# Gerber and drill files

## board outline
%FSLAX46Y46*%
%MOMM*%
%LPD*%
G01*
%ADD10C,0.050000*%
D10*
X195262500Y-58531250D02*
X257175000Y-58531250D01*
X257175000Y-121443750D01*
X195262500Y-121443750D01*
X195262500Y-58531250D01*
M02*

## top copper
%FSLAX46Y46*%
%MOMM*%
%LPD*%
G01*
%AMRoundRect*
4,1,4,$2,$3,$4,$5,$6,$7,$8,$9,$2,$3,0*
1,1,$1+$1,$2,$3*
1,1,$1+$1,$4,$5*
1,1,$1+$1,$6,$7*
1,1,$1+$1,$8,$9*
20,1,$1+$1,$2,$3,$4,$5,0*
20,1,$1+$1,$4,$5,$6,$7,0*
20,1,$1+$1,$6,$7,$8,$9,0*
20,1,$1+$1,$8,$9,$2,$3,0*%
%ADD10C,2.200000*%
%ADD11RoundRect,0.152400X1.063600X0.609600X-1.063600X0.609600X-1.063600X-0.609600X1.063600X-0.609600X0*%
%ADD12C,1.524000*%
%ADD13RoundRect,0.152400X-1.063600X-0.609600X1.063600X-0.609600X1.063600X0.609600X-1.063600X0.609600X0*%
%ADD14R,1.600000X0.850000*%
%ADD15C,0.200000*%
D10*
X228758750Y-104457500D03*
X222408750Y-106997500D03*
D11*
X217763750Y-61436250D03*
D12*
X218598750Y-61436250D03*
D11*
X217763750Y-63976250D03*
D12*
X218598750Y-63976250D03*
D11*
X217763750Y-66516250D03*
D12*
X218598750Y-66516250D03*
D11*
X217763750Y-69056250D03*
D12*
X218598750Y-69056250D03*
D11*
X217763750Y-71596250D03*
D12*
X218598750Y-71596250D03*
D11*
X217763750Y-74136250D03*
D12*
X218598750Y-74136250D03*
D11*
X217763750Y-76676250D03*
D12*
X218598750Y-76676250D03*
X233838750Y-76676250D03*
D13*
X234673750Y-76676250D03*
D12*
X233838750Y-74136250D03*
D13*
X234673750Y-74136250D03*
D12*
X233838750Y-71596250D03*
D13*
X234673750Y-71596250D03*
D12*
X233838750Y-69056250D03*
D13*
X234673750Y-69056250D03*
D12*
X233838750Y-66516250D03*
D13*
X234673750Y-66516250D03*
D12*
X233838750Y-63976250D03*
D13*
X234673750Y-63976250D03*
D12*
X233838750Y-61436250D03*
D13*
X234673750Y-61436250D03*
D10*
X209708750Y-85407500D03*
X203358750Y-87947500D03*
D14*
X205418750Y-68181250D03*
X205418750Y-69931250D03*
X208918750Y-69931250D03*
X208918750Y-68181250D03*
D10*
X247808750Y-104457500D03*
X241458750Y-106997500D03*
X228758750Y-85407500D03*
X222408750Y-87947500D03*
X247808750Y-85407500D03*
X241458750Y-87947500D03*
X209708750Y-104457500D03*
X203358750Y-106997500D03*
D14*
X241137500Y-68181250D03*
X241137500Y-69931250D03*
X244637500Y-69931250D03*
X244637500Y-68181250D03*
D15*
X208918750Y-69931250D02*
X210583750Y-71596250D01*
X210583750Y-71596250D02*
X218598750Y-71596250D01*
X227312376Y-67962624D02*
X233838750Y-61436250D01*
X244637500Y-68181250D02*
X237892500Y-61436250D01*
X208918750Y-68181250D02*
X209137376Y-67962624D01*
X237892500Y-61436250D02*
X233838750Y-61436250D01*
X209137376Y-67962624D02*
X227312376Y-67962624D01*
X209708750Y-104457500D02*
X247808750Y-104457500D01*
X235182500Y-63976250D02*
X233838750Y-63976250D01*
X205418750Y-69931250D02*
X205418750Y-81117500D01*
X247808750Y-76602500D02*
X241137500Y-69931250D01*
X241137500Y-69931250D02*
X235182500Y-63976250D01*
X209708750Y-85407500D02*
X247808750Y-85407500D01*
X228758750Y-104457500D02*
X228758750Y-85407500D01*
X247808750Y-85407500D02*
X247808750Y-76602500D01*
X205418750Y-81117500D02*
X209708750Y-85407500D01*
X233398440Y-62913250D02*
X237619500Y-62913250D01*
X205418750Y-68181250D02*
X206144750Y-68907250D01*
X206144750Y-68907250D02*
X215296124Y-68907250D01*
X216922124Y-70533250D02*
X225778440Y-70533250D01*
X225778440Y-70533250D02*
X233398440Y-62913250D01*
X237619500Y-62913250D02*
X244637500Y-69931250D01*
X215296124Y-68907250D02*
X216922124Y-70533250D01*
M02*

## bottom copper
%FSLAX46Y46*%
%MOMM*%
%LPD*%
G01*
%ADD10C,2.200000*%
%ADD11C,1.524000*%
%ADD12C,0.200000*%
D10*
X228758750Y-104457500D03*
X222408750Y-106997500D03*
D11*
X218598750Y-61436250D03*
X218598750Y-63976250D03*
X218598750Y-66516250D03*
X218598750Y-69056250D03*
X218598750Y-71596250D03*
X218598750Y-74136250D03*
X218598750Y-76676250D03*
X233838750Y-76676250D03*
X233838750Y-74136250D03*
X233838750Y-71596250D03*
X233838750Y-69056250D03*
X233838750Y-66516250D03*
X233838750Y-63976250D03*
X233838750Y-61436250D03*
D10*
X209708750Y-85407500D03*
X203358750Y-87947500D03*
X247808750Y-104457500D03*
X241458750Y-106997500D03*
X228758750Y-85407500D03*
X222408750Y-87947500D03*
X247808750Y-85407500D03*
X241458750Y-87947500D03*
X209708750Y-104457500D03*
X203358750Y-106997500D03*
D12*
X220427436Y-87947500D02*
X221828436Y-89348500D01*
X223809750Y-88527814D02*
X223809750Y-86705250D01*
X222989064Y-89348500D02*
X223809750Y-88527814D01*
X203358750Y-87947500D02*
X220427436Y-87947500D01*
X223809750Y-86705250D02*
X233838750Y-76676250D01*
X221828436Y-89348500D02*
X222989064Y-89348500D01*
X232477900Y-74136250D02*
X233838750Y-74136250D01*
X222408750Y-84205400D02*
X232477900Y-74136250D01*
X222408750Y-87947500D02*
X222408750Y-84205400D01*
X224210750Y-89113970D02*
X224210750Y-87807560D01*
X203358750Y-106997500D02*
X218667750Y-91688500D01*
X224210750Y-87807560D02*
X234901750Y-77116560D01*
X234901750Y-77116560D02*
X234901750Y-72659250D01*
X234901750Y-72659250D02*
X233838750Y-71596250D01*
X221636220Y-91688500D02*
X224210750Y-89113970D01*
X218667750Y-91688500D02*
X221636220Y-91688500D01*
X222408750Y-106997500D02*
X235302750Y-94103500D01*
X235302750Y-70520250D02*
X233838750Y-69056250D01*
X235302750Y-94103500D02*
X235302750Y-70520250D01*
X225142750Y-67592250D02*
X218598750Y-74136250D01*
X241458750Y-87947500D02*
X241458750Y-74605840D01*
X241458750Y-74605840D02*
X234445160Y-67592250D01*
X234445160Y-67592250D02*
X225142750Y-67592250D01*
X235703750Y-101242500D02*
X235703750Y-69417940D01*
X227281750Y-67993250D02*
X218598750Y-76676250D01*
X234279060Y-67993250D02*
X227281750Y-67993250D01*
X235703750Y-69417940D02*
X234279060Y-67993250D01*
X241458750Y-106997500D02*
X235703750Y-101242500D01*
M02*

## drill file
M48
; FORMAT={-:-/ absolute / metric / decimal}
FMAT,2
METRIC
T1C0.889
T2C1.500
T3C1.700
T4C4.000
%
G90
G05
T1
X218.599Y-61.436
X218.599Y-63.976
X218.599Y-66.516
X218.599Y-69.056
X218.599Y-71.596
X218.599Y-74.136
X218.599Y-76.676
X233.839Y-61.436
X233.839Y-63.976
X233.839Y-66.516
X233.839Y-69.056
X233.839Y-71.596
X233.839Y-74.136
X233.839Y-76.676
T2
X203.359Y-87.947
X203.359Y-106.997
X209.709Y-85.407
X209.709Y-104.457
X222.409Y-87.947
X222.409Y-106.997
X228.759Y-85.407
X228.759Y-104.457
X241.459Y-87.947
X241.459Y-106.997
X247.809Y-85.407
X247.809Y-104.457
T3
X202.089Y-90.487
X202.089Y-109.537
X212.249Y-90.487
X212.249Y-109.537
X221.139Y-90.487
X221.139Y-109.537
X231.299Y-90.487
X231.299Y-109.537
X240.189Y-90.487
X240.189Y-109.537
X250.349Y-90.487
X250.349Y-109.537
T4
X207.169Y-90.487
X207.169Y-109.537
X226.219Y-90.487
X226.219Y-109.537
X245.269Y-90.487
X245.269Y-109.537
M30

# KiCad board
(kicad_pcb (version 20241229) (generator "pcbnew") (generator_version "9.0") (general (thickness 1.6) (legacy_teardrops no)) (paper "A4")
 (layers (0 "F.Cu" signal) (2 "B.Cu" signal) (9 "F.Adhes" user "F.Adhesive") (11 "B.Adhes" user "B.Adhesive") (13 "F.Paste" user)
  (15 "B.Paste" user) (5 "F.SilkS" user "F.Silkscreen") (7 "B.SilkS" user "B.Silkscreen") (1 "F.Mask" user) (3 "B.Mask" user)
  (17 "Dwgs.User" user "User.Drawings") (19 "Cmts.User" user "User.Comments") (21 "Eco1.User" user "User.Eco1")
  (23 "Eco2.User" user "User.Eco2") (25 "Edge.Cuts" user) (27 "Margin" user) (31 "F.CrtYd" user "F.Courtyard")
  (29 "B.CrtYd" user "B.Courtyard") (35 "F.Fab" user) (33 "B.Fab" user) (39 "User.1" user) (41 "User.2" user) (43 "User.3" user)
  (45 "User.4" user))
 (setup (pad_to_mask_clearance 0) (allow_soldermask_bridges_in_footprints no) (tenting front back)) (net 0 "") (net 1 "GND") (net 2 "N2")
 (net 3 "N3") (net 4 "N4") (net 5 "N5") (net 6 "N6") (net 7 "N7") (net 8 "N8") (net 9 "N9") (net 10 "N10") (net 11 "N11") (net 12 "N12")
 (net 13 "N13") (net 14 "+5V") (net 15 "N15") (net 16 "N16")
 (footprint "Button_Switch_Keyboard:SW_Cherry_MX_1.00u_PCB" (layer "F.Cu") (at 228.75875 104.4575)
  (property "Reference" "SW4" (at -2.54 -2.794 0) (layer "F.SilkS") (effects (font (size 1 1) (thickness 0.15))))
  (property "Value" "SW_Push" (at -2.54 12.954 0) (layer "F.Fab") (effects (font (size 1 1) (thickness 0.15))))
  (pad "" np_thru_hole circle (at -7.62 5.08) (size 1.7 1.7) (drill 1.7) (layers "*.Cu" "*.Mask"))
  (pad "" np_thru_hole circle (at -2.54 5.08) (size 4 4) (drill 4) (layers "*.Cu" "*.Mask"))
  (pad "" np_thru_hole circle (at 2.54 5.08) (size 1.7 1.7) (drill 1.7) (layers "*.Cu" "*.Mask"))
  (pad "1" thru_hole circle (at 0 0) (size 2.2 2.2) (drill 1.5) (layers "*.Cu" "*.Mask") (remove_unused_layers no) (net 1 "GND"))
  (pad "2" thru_hole circle (at -6.35 2.54) (size 2.2 2.2) (drill 1.5) (layers "*.Cu" "*.Mask") (remove_unused_layers no) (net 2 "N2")))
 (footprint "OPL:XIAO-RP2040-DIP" (layer "F.Cu") (at 226.21875 69.05625)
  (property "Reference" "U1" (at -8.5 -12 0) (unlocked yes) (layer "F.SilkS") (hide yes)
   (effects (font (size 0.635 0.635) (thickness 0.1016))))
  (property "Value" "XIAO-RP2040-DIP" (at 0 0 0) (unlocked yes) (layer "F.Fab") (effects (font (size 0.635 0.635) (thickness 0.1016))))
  (pad "1" smd roundrect (at -8.455 -7.62 180) (size 2.432 1.524) (layers "F.Cu" "F.Mask") (roundrect_rratio 0.1) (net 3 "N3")
   (thermal_bridge_angle 45))
  (pad "1" thru_hole circle (at -7.62 -7.62 180) (size 1.524 1.524) (drill 0.889) (layers "*.Cu" "*.Mask") (remove_unused_layers no)
   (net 3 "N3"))
  (pad "2" smd roundrect (at -8.455 -5.08 180) (size 2.432 1.524) (layers "F.Cu" "F.Mask") (roundrect_rratio 0.1) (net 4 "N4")
   (thermal_bridge_angle 45))
  (pad "2" thru_hole circle (at -7.62 -5.08 180) (size 1.524 1.524) (drill 0.889) (layers "*.Cu" "*.Mask") (remove_unused_layers no)
   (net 4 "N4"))
  (pad "3" smd roundrect (at -8.455 -2.54 180) (size 2.432 1.524) (layers "F.Cu" "F.Mask") (roundrect_rratio 0.1) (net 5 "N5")
   (thermal_bridge_angle 45))
  (pad "3" thru_hole circle (at -7.62 -2.54 180) (size 1.524 1.524) (drill 0.889) (layers "*.Cu" "*.Mask") (remove_unused_layers no)
   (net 5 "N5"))
  (pad "4" smd roundrect (at -8.455 0 180) (size 2.432 1.524) (layers "F.Cu" "F.Mask") (roundrect_rratio 0.1) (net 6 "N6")
   (thermal_bridge_angle 45))
  (pad "4" thru_hole circle (at -7.62 0 180) (size 1.524 1.524) (drill 0.889) (layers "*.Cu" "*.Mask") (remove_unused_layers no)
   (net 6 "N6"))
  (pad "5" smd roundrect (at -8.455 2.54 180) (size 2.432 1.524) (layers "F.Cu" "F.Mask") (roundrect_rratio 0.1) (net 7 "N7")
   (thermal_bridge_angle 45))
  (pad "5" thru_hole circle (at -7.62 2.54 180) (size 1.524 1.524) (drill 0.889) (layers "*.Cu" "*.Mask") (remove_unused_layers no)
   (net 7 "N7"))
  (pad "6" smd roundrect (at -8.455 5.08 180) (size 2.432 1.524) (layers "F.Cu" "F.Mask") (roundrect_rratio 0.1) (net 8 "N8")
   (thermal_bridge_angle 45))
  (pad "6" thru_hole circle (at -7.62 5.08 180) (size 1.524 1.524) (drill 0.889) (layers "*.Cu" "*.Mask") (remove_unused_layers no)
   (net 8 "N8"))
  (pad "7" smd roundrect (at -8.455 7.62 180) (size 2.432 1.524) (layers "F.Cu" "F.Mask") (roundrect_rratio 0.1) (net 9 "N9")
   (thermal_bridge_angle 45))
  (pad "7" thru_hole circle (at -7.62 7.62 180) (size 1.524 1.524) (drill 0.889) (layers "*.Cu" "*.Mask") (remove_unused_layers no)
   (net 9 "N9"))
  (pad "8" thru_hole circle (at 7.62 7.62) (size 1.524 1.524) (drill 0.889) (layers "*.Cu" "*.Mask") (remove_unused_layers no)
   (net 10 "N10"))
  (pad "8" smd roundrect (at 8.455 7.62) (size 2.432 1.524) (layers "F.Cu" "F.Mask") (roundrect_rratio 0.1) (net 10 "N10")
   (thermal_bridge_angle 45))
  (pad "9" thru_hole circle (at 7.62 5.08) (size 1.524 1.524) (drill 0.889) (layers "*.Cu" "*.Mask") (remove_unused_layers no)
   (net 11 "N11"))
  (pad "9" smd roundrect (at 8.455 5.08) (size 2.432 1.524) (layers "F.Cu" "F.Mask") (roundrect_rratio 0.1) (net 11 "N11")
   (thermal_bridge_angle 45))
  (pad "10" thru_hole circle (at 7.62 2.54) (size 1.524 1.524) (drill 0.889) (layers "*.Cu" "*.Mask") (remove_unused_layers no)
   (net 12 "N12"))
  (pad "10" smd roundrect (at 8.455 2.54) (size 2.432 1.524) (layers "F.Cu" "F.Mask") (roundrect_rratio 0.1) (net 12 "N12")
   (thermal_bridge_angle 45))
  (pad "11" thru_hole circle (at 7.62 0) (size 1.524 1.524) (drill 0.889) (layers "*.Cu" "*.Mask") (remove_unused_layers no) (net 2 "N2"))
  (pad "11" smd roundrect (at 8.455 0) (size 2.432 1.524) (layers "F.Cu" "F.Mask") (roundrect_rratio 0.1) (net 2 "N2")
   (thermal_bridge_angle 45))
  (pad "12" thru_hole circle (at 7.62 -2.54) (size 1.524 1.524) (drill 0.889) (layers "*.Cu" "*.Mask") (remove_unused_layers no)
   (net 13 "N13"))
  (pad "12" smd roundrect (at 8.455 -2.54) (size 2.432 1.524) (layers "F.Cu" "F.Mask") (roundrect_rratio 0.1) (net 13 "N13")
   (thermal_bridge_angle 45))
  (pad "13" thru_hole circle (at 7.62 -5.08) (size 1.524 1.524) (drill 0.889) (layers "*.Cu" "*.Mask") (remove_unused_layers no)
   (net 1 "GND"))
  (pad "13" smd roundrect (at 8.455 -5.08) (size 2.432 1.524) (layers "F.Cu" "F.Mask") (roundrect_rratio 0.1) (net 1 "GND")
   (thermal_bridge_angle 45))
  (pad "14" thru_hole circle (at 7.62 -7.62) (size 1.524 1.524) (drill 0.889) (layers "*.Cu" "*.Mask") (remove_unused_layers no)
   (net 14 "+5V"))
  (pad "14" smd roundrect (at 8.455 -7.62) (size 2.432 1.524) (layers "F.Cu" "F.Mask") (roundrect_rratio 0.1) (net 14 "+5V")
   (thermal_bridge_angle 45)))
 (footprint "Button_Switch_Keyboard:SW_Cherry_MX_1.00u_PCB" (layer "F.Cu") (at 209.70875 85.4075)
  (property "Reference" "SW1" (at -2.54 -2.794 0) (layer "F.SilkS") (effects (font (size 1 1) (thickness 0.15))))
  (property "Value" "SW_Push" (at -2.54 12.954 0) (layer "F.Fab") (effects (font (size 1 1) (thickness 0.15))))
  (pad "" np_thru_hole circle (at -7.62 5.08) (size 1.7 1.7) (drill 1.7) (layers "*.Cu" "*.Mask"))
  (pad "" np_thru_hole circle (at -2.54 5.08) (size 4 4) (drill 4) (layers "*.Cu" "*.Mask"))
  (pad "" np_thru_hole circle (at 2.54 5.08) (size 1.7 1.7) (drill 1.7) (layers "*.Cu" "*.Mask"))
  (pad "1" thru_hole circle (at 0 0) (size 2.2 2.2) (drill 1.5) (layers "*.Cu" "*.Mask") (remove_unused_layers no) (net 1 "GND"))
  (pad "2" thru_hole circle (at -6.35 2.54) (size 2.2 2.2) (drill 1.5) (layers "*.Cu" "*.Mask") (remove_unused_layers no) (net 10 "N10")))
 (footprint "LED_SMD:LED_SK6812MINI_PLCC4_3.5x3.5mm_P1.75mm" (layer "F.Cu") (at 207.16875 69.05625)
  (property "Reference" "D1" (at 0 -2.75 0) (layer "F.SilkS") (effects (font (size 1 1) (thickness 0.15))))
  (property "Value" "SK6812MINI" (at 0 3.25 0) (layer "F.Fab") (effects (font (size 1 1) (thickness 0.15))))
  (pad "1" smd rect (at -1.75 -0.875) (size 1.6 0.85) (layers "F.Cu" "F.Mask" "F.Paste") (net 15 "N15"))
  (pad "2" smd rect (at -1.75 0.875) (size 1.6 0.85) (layers "F.Cu" "F.Mask" "F.Paste") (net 1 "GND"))
  (pad "3" smd rect (at 1.75 0.875) (size 1.6 0.85) (layers "F.Cu" "F.Mask" "F.Paste") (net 7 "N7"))
  (pad "4" smd rect (at 1.75 -0.875) (size 1.6 0.85) (layers "F.Cu" "F.Mask" "F.Paste") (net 14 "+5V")))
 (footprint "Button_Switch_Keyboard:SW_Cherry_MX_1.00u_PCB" (layer "F.Cu") (at 247.80875 104.4575)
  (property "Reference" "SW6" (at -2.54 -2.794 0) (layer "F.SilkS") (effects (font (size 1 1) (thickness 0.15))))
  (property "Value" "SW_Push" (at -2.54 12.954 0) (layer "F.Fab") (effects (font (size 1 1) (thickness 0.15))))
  (pad "" np_thru_hole circle (at -7.62 5.08) (size 1.7 1.7) (drill 1.7) (layers "*.Cu" "*.Mask"))
  (pad "" np_thru_hole circle (at -2.54 5.08) (size 4 4) (drill 4) (layers "*.Cu" "*.Mask"))
  (pad "" np_thru_hole circle (at 2.54 5.08) (size 1.7 1.7) (drill 1.7) (layers "*.Cu" "*.Mask"))
  (pad "1" thru_hole circle (at 0 0) (size 2.2 2.2) (drill 1.5) (layers "*.Cu" "*.Mask") (remove_unused_layers no) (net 1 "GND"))
  (pad "2" thru_hole circle (at -6.35 2.54) (size 2.2 2.2) (drill 1.5) (layers "*.Cu" "*.Mask") (remove_unused_layers no) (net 9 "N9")))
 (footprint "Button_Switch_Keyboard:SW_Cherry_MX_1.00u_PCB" (layer "F.Cu") (at 228.75875 85.4075)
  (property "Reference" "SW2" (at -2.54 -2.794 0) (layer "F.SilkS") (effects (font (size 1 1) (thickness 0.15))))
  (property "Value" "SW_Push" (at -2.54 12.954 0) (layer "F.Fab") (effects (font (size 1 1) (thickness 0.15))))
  (pad "" np_thru_hole circle (at -7.62 5.08) (size 1.7 1.7) (drill 1.7) (layers "*.Cu" "*.Mask"))
  (pad "" np_thru_hole circle (at -2.54 5.08) (size 4 4) (drill 4) (layers "*.Cu" "*.Mask"))
  (pad "" np_thru_hole circle (at 2.54 5.08) (size 1.7 1.7) (drill 1.7) (layers "*.Cu" "*.Mask"))
  (pad "1" thru_hole circle (at 0 0) (size 2.2 2.2) (drill 1.5) (layers "*.Cu" "*.Mask") (remove_unused_layers no) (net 1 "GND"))
  (pad "2" thru_hole circle (at -6.35 2.54) (size 2.2 2.2) (drill 1.5) (layers "*.Cu" "*.Mask") (remove_unused_layers no) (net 11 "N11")))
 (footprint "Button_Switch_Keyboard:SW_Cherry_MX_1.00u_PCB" (layer "F.Cu") (at 247.80875 85.4075)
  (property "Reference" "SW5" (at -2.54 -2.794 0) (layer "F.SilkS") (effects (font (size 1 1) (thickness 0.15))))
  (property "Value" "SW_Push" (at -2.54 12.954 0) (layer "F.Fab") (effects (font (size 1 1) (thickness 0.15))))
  (pad "" np_thru_hole circle (at -7.62 5.08) (size 1.7 1.7) (drill 1.7) (layers "*.Cu" "*.Mask"))
  (pad "" np_thru_hole circle (at -2.54 5.08) (size 4 4) (drill 4) (layers "*.Cu" "*.Mask"))
  (pad "" np_thru_hole circle (at 2.54 5.08) (size 1.7 1.7) (drill 1.7) (layers "*.Cu" "*.Mask"))
  (pad "1" thru_hole circle (at 0 0) (size 2.2 2.2) (drill 1.5) (layers "*.Cu" "*.Mask") (remove_unused_layers no) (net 1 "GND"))
  (pad "2" thru_hole circle (at -6.35 2.54) (size 2.2 2.2) (drill 1.5) (layers "*.Cu" "*.Mask") (remove_unused_layers no) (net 8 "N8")))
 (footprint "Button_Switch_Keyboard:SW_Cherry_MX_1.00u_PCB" (layer "F.Cu") (at 209.70875 104.4575)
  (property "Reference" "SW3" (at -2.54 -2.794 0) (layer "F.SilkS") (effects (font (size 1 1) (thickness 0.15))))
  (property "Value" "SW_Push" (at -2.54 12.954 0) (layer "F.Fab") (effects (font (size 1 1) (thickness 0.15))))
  (pad "" np_thru_hole circle (at -7.62 5.08) (size 1.7 1.7) (drill 1.7) (layers "*.Cu" "*.Mask"))
  (pad "" np_thru_hole circle (at -2.54 5.08) (size 4 4) (drill 4) (layers "*.Cu" "*.Mask"))
  (pad "" np_thru_hole circle (at 2.54 5.08) (size 1.7 1.7) (drill 1.7) (layers "*.Cu" "*.Mask"))
  (pad "1" thru_hole circle (at 0 0) (size 2.2 2.2) (drill 1.5) (layers "*.Cu" "*.Mask") (remove_unused_layers no) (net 1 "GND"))
  (pad "2" thru_hole circle (at -6.35 2.54) (size 2.2 2.2) (drill 1.5) (layers "*.Cu" "*.Mask") (remove_unused_layers no) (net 12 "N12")))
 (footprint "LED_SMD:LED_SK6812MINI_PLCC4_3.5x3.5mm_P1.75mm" (layer "F.Cu") (at 242.8875 69.05625)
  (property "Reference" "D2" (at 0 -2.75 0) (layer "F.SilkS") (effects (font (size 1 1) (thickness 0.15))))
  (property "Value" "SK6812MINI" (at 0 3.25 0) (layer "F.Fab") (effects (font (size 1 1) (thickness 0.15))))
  (pad "1" smd rect (at -1.75 -0.875) (size 1.6 0.85) (layers "F.Cu" "F.Mask" "F.Paste") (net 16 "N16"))
  (pad "2" smd rect (at -1.75 0.875) (size 1.6 0.85) (layers "F.Cu" "F.Mask" "F.Paste") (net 1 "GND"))
  (pad "3" smd rect (at 1.75 0.875) (size 1.6 0.85) (layers "F.Cu" "F.Mask" "F.Paste") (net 15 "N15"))
  (pad "4" smd rect (at 1.75 -0.875) (size 1.6 0.85) (layers "F.Cu" "F.Mask" "F.Paste") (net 14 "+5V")))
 (gr_rect (start 195.2625 58.53125) (end 257.175 121.44375) (stroke (width 0.05) (type default)) (fill no) (layer "Edge.Cuts"))
 (segment (start 208.91875 69.93125) (end 210.58375 71.59625) (width 0.2) (layer "F.Cu") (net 7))
 (segment (start 210.58375 71.59625) (end 218.59875 71.59625) (width 0.2) (layer "F.Cu") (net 7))
 (segment (start 227.312376 67.962624) (end 233.83875 61.43625) (width 0.2) (layer "F.Cu") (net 14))
 (segment (start 244.6375 68.18125) (end 237.8925 61.43625) (width 0.2) (layer "F.Cu") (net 14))
 (segment (start 208.91875 68.18125) (end 209.137376 67.962624) (width 0.2) (layer "F.Cu") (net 14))
 (segment (start 237.8925 61.43625) (end 233.83875 61.43625) (width 0.2) (layer "F.Cu") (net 14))
 (segment (start 209.137376 67.962624) (end 227.312376 67.962624) (width 0.2) (layer "F.Cu") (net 14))
 (segment (start 209.70875 104.4575) (end 247.80875 104.4575) (width 0.2) (layer "F.Cu") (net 1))
 (segment (start 235.1825 63.97625) (end 233.83875 63.97625) (width 0.2) (layer "F.Cu") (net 1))
 (segment (start 205.41875 69.93125) (end 205.41875 81.1175) (width 0.2) (layer "F.Cu") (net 1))
 (segment (start 247.80875 76.6025) (end 241.1375 69.93125) (width 0.2) (layer "F.Cu") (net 1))
 (segment (start 241.1375 69.93125) (end 235.1825 63.97625) (width 0.2) (layer "F.Cu") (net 1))
 (segment (start 209.70875 85.4075) (end 247.80875 85.4075) (width 0.2) (layer "F.Cu") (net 1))
 (segment (start 228.75875 104.4575) (end 228.75875 85.4075) (width 0.2) (layer "F.Cu") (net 1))
 (segment (start 247.80875 85.4075) (end 247.80875 76.6025) (width 0.2) (layer "F.Cu") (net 1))
 (segment (start 205.41875 81.1175) (end 209.70875 85.4075) (width 0.2) (layer "F.Cu") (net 1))
 (segment (start 233.39844 62.91325) (end 237.6195 62.91325) (width 0.2) (layer "F.Cu") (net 15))
 (segment (start 205.41875 68.18125) (end 206.14475 68.90725) (width 0.2) (layer "F.Cu") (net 15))
 (segment (start 206.14475 68.90725) (end 215.296124 68.90725) (width 0.2) (layer "F.Cu") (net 15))
 (segment (start 216.922124 70.53325) (end 225.77844 70.53325) (width 0.2) (layer "F.Cu") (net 15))
 (segment (start 225.77844 70.53325) (end 233.39844 62.91325) (width 0.2) (layer "F.Cu") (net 15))
 (segment (start 237.6195 62.91325) (end 244.6375 69.93125) (width 0.2) (layer "F.Cu") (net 15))
 (segment (start 215.296124 68.90725) (end 216.922124 70.53325) (width 0.2) (layer "F.Cu") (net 15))
 (segment (start 220.427436 87.9475) (end 221.828436 89.3485) (width 0.2) (layer "B.Cu") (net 10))
 (segment (start 223.80975 88.527814) (end 223.80975 86.70525) (width 0.2) (layer "B.Cu") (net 10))
 (segment (start 222.989064 89.3485) (end 223.80975 88.527814) (width 0.2) (layer "B.Cu") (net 10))
 (segment (start 203.35875 87.9475) (end 220.427436 87.9475) (width 0.2) (layer "B.Cu") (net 10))
 (segment (start 223.80975 86.70525) (end 233.83875 76.67625) (width 0.2) (layer "B.Cu") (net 10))
 (segment (start 221.828436 89.3485) (end 222.989064 89.3485) (width 0.2) (layer "B.Cu") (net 10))
 (segment (start 232.4779 74.13625) (end 233.83875 74.13625) (width 0.2) (layer "B.Cu") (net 11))
 (segment (start 222.40875 84.2054) (end 232.4779 74.13625) (width 0.2) (layer "B.Cu") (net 11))
 (segment (start 222.40875 87.9475) (end 222.40875 84.2054) (width 0.2) (layer "B.Cu") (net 11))
 (segment (start 224.21075 89.11397) (end 224.21075 87.80756) (width 0.2) (layer "B.Cu") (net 12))
 (segment (start 203.35875 106.9975) (end 218.66775 91.6885) (width 0.2) (layer "B.Cu") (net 12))
 (segment (start 224.21075 87.80756) (end 234.90175 77.11656) (width 0.2) (layer "B.Cu") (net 12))
 (segment (start 234.90175 77.11656) (end 234.90175 72.65925) (width 0.2) (layer "B.Cu") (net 12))
 (segment (start 234.90175 72.65925) (end 233.83875 71.59625) (width 0.2) (layer "B.Cu") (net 12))
 (segment (start 221.63622 91.6885) (end 224.21075 89.11397) (width 0.2) (layer "B.Cu") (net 12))
 (segment (start 218.66775 91.6885) (end 221.63622 91.6885) (width 0.2) (layer "B.Cu") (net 12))
 (segment (start 222.40875 106.9975) (end 235.30275 94.1035) (width 0.2) (layer "B.Cu") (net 2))
 (segment (start 235.30275 70.52025) (end 233.83875 69.05625) (width 0.2) (layer "B.Cu") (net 2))
 (segment (start 235.30275 94.1035) (end 235.30275 70.52025) (width 0.2) (layer "B.Cu") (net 2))
 (segment (start 225.14275 67.59225) (end 218.59875 74.13625) (width 0.2) (layer "B.Cu") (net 8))
 (segment (start 241.45875 87.9475) (end 241.45875 74.60584) (width 0.2) (layer "B.Cu") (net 8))
 (segment (start 241.45875 74.60584) (end 234.44516 67.59225) (width 0.2) (layer "B.Cu") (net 8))
 (segment (start 234.44516 67.59225) (end 225.14275 67.59225) (width 0.2) (layer "B.Cu") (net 8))
 (segment (start 235.70375 101.2425) (end 235.70375 69.41794) (width 0.2) (layer "B.Cu") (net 9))
 (segment (start 227.28175 67.99325) (end 218.59875 76.67625) (width 0.2) (layer "B.Cu") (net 9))
 (segment (start 234.27906 67.99325) (end 227.28175 67.99325) (width 0.2) (layer "B.Cu") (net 9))
 (segment (start 235.70375 69.41794) (end 234.27906 67.99325) (width 0.2) (layer "B.Cu") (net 9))
 (segment (start 241.45875 106.9975) (end 235.70375 101.2425) (width 0.2) (layer "B.Cu") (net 9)))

